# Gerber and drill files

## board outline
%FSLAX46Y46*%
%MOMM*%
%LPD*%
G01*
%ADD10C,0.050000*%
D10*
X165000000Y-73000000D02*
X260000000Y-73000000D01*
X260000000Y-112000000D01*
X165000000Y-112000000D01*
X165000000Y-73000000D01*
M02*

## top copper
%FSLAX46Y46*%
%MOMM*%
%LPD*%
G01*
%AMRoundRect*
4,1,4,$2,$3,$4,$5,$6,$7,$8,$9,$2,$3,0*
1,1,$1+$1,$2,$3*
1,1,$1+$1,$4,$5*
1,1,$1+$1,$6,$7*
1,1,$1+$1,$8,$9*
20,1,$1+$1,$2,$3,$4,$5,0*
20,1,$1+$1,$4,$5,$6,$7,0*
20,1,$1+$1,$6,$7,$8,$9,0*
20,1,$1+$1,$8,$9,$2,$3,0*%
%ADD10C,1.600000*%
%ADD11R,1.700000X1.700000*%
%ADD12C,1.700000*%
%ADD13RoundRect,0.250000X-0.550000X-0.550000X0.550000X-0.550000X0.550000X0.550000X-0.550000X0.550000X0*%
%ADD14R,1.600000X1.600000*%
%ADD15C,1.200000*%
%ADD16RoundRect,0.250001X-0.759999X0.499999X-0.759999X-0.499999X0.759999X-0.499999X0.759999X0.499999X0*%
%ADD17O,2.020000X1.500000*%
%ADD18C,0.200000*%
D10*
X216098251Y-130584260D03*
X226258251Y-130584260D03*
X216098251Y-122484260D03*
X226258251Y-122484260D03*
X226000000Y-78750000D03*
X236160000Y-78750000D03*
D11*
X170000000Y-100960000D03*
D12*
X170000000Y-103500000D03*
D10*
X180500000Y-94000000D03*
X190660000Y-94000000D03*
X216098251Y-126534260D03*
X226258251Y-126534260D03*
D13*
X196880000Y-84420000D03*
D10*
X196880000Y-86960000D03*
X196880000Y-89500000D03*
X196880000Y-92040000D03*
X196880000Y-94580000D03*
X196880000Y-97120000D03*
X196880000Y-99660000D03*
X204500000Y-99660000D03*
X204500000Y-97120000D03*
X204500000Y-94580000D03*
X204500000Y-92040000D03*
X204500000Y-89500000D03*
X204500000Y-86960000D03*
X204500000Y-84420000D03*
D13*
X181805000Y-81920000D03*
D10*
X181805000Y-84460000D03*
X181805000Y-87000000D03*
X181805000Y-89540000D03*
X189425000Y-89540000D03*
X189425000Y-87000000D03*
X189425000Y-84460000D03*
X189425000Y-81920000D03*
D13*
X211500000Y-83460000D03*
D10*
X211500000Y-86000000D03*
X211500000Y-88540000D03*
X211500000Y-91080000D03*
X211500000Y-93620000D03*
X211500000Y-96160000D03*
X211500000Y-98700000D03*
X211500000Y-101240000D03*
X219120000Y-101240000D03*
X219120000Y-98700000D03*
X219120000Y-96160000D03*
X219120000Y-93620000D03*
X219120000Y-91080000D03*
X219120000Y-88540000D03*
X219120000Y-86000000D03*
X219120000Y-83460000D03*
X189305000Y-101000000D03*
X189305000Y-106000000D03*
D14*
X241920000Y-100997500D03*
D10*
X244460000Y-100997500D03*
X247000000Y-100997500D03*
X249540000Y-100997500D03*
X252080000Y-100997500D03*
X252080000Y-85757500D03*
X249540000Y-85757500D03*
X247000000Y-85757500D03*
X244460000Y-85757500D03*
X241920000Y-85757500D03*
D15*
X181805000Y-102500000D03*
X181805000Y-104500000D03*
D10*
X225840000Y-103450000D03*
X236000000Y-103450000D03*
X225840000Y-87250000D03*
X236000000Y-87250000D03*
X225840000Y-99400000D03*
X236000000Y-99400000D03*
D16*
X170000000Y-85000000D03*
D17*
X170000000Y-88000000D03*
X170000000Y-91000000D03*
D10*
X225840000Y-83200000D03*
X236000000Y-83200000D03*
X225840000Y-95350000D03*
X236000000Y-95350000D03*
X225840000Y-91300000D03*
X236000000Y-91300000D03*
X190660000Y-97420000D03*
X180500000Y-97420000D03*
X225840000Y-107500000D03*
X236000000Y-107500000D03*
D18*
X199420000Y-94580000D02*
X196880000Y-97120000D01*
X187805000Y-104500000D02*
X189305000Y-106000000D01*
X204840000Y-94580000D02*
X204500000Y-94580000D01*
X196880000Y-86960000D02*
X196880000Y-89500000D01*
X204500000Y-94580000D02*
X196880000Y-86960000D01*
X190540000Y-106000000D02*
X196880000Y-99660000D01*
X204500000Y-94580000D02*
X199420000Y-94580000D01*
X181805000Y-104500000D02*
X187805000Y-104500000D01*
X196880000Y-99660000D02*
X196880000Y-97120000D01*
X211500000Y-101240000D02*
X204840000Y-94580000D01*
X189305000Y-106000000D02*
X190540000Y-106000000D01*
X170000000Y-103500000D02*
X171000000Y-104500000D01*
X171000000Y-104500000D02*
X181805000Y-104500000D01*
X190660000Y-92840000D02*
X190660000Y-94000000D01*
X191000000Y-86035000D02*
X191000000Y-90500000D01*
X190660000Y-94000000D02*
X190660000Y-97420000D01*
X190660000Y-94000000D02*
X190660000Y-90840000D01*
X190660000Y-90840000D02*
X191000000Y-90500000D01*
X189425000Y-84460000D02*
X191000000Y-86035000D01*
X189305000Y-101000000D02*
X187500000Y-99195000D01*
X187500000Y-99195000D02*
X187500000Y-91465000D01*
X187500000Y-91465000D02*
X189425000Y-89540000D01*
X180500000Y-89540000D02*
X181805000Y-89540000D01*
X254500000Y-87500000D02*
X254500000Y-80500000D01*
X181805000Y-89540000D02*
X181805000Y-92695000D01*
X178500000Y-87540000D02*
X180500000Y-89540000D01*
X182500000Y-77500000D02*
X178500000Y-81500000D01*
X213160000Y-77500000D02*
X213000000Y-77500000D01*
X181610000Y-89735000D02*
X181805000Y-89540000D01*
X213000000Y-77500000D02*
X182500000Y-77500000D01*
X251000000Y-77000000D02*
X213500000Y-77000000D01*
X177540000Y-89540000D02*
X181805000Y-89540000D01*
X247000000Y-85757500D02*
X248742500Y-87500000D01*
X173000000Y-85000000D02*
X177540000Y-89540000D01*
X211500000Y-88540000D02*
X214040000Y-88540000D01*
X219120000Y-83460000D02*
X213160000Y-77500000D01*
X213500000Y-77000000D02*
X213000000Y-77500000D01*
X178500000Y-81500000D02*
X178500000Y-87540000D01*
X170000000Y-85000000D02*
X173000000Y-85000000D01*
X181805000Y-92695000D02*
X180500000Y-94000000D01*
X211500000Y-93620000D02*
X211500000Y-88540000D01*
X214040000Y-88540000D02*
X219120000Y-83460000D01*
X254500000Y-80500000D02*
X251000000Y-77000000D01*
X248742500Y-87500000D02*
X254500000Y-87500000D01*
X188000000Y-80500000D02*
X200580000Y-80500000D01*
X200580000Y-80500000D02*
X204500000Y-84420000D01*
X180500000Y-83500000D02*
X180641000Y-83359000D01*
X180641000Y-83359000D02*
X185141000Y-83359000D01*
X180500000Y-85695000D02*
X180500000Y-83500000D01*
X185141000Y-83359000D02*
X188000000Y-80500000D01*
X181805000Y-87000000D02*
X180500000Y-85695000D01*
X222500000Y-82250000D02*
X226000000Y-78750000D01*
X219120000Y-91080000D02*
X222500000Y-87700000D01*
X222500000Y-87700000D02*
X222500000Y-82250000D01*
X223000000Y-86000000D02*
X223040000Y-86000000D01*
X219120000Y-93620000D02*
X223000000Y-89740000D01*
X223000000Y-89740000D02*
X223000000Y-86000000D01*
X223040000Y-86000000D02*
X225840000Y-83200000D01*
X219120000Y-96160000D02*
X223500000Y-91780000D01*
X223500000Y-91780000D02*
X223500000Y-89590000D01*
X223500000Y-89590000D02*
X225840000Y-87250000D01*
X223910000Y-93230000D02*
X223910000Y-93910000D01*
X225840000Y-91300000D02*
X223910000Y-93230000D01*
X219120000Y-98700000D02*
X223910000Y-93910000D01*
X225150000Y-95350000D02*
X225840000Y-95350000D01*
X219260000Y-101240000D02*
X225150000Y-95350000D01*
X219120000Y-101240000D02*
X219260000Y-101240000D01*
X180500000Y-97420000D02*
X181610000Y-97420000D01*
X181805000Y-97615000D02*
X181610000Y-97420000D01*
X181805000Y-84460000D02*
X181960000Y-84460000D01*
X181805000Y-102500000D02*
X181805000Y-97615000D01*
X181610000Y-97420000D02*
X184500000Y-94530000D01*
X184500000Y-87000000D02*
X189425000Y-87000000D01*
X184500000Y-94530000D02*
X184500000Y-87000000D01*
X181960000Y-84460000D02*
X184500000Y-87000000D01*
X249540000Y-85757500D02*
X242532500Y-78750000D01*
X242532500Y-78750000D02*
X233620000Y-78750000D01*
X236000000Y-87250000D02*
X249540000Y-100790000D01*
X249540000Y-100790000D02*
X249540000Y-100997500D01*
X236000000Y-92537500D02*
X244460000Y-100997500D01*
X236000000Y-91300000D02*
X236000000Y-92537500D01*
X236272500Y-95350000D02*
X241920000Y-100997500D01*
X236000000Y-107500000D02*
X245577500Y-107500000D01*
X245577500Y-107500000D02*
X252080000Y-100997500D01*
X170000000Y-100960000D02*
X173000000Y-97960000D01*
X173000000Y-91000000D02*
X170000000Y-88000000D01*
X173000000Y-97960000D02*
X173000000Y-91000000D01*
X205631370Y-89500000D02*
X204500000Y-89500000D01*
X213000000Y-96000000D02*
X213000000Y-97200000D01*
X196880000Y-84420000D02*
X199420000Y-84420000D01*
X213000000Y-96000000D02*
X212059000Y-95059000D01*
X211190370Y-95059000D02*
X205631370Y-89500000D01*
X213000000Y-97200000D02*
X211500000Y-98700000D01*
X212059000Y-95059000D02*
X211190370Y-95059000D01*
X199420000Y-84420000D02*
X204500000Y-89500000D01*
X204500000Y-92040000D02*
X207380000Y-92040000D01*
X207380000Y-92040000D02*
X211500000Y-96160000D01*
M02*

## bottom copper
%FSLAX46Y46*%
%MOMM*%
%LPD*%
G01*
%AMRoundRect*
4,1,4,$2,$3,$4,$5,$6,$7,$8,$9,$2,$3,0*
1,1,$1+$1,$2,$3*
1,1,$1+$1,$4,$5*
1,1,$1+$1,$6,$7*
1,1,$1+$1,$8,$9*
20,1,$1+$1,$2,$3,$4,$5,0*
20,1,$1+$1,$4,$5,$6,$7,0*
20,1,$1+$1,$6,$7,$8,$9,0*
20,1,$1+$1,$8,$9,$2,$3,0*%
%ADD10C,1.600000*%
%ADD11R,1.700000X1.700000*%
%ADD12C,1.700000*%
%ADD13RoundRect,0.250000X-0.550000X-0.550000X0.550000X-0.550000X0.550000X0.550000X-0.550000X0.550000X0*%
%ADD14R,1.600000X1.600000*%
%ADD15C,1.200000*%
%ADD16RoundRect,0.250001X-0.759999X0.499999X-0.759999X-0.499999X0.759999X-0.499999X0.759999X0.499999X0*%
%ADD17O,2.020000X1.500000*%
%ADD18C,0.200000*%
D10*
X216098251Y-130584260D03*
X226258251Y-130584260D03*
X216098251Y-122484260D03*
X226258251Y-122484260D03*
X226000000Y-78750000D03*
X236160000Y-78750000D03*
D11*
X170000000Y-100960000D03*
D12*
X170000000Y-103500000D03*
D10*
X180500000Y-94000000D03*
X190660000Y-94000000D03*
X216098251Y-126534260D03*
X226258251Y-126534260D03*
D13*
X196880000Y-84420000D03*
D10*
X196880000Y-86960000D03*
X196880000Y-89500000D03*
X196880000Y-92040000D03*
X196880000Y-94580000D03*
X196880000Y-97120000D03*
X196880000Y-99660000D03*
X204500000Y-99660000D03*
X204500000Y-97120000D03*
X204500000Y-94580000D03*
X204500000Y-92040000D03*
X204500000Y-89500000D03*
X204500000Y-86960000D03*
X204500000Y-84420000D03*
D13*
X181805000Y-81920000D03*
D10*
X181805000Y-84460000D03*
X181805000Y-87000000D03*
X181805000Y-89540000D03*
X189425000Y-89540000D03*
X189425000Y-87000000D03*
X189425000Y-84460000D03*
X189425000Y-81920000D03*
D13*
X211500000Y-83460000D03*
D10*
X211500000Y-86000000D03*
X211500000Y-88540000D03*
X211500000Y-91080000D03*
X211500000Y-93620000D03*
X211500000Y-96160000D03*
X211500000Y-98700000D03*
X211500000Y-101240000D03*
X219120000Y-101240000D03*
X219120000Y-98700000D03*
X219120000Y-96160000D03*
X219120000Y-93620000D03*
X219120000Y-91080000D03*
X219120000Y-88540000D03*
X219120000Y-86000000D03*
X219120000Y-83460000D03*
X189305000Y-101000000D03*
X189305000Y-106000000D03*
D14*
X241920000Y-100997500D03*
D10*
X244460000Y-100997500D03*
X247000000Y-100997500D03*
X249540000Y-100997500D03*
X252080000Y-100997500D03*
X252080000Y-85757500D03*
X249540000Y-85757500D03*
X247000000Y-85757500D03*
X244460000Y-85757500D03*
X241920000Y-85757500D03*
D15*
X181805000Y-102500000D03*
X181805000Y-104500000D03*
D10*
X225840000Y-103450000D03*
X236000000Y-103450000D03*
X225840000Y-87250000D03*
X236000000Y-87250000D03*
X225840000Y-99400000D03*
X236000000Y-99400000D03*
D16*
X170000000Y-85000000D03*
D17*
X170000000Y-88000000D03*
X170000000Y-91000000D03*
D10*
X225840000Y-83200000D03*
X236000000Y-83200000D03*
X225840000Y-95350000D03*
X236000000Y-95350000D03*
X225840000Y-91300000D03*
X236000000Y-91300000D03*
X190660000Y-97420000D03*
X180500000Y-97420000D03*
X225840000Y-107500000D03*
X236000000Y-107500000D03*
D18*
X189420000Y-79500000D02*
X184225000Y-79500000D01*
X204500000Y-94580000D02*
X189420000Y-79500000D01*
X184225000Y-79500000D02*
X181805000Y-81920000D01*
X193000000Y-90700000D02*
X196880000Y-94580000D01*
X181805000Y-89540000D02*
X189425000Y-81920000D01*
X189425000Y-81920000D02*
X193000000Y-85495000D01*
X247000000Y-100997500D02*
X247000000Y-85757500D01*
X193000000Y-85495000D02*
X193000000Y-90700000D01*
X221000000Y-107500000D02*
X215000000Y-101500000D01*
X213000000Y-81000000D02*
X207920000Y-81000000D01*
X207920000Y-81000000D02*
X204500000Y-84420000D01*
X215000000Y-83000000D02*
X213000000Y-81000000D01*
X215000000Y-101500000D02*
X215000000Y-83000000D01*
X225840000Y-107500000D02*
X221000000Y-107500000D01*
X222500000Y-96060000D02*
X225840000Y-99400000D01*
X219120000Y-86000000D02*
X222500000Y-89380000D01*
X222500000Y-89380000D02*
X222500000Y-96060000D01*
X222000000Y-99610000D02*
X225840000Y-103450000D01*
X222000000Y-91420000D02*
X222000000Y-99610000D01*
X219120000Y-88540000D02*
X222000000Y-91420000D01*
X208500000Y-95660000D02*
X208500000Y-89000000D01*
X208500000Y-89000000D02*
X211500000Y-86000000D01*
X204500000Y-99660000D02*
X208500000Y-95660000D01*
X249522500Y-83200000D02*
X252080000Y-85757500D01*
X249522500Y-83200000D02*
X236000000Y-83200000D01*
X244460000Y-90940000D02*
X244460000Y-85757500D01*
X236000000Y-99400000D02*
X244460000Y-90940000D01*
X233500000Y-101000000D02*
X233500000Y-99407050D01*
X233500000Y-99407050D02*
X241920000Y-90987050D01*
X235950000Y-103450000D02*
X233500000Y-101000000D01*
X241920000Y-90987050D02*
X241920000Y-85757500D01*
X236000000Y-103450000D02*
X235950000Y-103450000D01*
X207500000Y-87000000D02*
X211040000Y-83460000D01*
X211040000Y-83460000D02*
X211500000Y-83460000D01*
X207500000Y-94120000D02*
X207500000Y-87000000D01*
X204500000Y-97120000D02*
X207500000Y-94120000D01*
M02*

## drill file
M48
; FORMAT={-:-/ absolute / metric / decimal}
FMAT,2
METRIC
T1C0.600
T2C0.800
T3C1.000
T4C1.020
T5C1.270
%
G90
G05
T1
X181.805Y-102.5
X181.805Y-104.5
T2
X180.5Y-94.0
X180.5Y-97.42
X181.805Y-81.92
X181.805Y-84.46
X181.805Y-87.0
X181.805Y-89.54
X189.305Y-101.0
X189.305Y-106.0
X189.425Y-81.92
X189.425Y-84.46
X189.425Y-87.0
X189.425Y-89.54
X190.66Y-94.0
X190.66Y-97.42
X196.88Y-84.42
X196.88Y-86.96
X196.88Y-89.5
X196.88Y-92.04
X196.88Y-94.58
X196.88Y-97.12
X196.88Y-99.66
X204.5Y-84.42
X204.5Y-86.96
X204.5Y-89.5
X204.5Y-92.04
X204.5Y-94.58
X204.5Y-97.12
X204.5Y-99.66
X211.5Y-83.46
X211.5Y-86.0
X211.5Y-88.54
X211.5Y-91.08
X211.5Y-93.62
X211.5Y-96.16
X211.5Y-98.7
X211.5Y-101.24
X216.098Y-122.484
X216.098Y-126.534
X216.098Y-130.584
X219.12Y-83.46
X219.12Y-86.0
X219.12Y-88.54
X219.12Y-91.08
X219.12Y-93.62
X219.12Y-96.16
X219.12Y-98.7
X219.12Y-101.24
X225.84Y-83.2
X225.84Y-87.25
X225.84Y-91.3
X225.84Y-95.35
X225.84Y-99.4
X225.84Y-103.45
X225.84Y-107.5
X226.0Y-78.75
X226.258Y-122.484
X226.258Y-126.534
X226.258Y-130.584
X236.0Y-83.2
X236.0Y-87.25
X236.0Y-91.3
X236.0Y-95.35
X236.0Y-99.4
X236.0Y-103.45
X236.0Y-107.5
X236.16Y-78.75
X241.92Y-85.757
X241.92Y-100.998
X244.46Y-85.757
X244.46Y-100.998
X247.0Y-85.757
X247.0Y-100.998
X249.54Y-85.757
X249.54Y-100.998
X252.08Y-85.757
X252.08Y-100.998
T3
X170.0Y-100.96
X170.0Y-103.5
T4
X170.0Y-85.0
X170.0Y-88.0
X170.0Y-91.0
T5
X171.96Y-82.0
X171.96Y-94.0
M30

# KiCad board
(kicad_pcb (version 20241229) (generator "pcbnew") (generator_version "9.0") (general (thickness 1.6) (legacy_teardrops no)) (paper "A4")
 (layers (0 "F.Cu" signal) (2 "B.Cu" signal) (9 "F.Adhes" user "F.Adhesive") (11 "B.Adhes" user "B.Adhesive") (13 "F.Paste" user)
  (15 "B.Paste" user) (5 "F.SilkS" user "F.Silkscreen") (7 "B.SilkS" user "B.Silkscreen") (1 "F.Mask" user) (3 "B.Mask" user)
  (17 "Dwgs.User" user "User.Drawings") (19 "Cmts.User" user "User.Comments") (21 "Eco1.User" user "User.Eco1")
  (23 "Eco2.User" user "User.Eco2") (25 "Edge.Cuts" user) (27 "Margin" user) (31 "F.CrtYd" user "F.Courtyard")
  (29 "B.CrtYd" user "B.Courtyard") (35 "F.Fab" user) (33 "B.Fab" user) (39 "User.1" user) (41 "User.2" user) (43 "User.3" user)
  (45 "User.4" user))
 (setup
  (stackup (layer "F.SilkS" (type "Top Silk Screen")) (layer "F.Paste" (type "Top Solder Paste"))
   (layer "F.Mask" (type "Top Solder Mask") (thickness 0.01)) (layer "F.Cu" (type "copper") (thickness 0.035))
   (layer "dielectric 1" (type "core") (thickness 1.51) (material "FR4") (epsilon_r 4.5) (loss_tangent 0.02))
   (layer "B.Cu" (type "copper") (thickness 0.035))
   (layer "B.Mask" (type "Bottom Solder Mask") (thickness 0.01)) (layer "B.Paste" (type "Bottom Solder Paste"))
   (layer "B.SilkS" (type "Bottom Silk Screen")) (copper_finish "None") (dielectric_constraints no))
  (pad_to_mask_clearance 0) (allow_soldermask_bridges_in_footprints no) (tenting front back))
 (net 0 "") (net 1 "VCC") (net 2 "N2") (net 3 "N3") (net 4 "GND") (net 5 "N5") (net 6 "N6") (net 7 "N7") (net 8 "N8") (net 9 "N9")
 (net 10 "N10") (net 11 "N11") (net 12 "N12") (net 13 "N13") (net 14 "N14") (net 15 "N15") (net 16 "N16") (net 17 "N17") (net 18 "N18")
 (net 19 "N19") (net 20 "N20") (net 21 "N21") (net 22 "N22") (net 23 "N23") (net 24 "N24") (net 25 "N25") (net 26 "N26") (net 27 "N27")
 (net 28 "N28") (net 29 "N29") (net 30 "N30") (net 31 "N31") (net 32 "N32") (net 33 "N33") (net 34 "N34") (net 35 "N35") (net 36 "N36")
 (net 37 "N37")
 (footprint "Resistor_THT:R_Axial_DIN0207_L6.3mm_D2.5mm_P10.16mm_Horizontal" (layer "F.Cu") (at 216.098251 130.58426)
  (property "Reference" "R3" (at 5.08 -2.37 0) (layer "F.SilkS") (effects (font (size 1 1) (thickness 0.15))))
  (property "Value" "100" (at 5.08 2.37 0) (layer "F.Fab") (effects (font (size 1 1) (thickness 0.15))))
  (pad "1" thru_hole circle (at 0 0) (size 1.6 1.6) (drill 0.8) (layers "*.Cu" "*.Mask") (remove_unused_layers no) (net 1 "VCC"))
  (pad "2" thru_hole circle (at 10.16 0) (size 1.6 1.6) (drill 0.8) (layers "*.Cu" "*.Mask") (remove_unused_layers no) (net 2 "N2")))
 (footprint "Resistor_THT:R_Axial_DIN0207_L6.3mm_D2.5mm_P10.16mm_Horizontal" (layer "F.Cu") (at 216.098251 122.48426)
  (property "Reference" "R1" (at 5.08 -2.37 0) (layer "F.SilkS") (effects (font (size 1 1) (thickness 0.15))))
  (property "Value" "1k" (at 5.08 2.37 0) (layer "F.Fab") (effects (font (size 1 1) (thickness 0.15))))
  (pad "1" thru_hole circle (at 0 0) (size 1.6 1.6) (drill 0.8) (layers "*.Cu" "*.Mask") (remove_unused_layers no) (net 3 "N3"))
  (pad "2" thru_hole circle (at 10.16 0) (size 1.6 1.6) (drill 0.8) (layers "*.Cu" "*.Mask") (remove_unused_layers no) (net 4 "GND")))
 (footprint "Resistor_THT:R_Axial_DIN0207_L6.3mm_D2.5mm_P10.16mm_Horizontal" (layer "F.Cu") (at 226 78.75)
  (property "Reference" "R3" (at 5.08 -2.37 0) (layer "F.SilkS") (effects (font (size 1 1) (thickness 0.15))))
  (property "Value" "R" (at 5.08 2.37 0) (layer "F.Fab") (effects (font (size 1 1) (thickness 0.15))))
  (pad "1" thru_hole circle (at 0 0) (size 1.6 1.6) (drill 0.8) (layers "*.Cu" "*.Mask") (remove_unused_layers no) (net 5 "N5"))
  (pad "2" thru_hole circle (at 10.16 0) (size 1.6 1.6) (drill 0.8) (layers "*.Cu" "*.Mask") (remove_unused_layers no) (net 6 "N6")))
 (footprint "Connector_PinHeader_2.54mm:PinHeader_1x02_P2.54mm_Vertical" (layer "F.Cu") (at 170 100.96)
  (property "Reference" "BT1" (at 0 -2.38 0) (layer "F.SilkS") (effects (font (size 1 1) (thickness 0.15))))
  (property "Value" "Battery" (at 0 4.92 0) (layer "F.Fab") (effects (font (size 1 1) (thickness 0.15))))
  (pad "1" thru_hole rect (at 0 0) (size 1.7 1.7) (drill 1) (layers "*.Cu" "*.Mask") (remove_unused_layers no) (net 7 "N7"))
  (pad "2" thru_hole circle (at 0 2.54) (size 1.7 1.7) (drill 1) (layers "*.Cu" "*.Mask") (remove_unused_layers no) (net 4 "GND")))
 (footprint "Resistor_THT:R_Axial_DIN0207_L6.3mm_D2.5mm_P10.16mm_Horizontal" (layer "F.Cu") (at 180.5 94)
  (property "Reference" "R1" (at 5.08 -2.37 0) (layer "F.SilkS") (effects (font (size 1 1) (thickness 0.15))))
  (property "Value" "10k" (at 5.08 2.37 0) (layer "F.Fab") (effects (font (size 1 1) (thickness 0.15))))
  (pad "1" thru_hole circle (at 0 0) (size 1.6 1.6) (drill 0.8) (layers "*.Cu" "*.Mask") (remove_unused_layers no) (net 1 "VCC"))
  (pad "2" thru_hole circle (at 10.16 0) (size 1.6 1.6) (drill 0.8) (layers "*.Cu" "*.Mask") (remove_unused_layers no) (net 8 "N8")))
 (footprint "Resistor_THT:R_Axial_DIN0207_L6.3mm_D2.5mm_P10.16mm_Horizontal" (layer "F.Cu") (at 216.098251 126.53426)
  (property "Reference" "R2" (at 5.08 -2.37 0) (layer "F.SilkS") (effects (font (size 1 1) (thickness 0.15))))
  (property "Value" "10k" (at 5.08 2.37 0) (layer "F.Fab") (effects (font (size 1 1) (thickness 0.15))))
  (pad "1" thru_hole circle (at 0 0) (size 1.6 1.6) (drill 0.8) (layers "*.Cu" "*.Mask") (remove_unused_layers no) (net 1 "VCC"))
  (pad "2" thru_hole circle (at 10.16 0) (size 1.6 1.6) (drill 0.8) (layers "*.Cu" "*.Mask") (remove_unused_layers no) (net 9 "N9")))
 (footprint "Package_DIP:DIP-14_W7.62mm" (layer "F.Cu") (at 196.88 84.42)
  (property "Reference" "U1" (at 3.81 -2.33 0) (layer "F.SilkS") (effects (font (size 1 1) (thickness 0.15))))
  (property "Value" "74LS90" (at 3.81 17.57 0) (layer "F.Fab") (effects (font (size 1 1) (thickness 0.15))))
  (pad "1" thru_hole roundrect (at 0 0) (size 1.6 1.6) (drill 0.8) (layers "*.Cu" "*.Mask") (remove_unused_layers no)
   (roundrect_rratio 0.15625) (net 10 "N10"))
  (pad "2" thru_hole circle (at 0 2.54) (size 1.6 1.6) (drill 0.8) (layers "*.Cu" "*.Mask") (remove_unused_layers no) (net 4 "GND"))
  (pad "3" thru_hole circle (at 0 5.08) (size 1.6 1.6) (drill 0.8) (layers "*.Cu" "*.Mask") (remove_unused_layers no) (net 4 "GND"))
  (pad "4" thru_hole circle (at 0 7.62) (size 1.6 1.6) (drill 0.8) (layers "*.Cu" "*.Mask") (remove_unused_layers no))
  (pad "5" thru_hole circle (at 0 10.16) (size 1.6 1.6) (drill 0.8) (layers "*.Cu" "*.Mask") (remove_unused_layers no) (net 1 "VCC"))
  (pad "6" thru_hole circle (at 0 12.7) (size 1.6 1.6) (drill 0.8) (layers "*.Cu" "*.Mask") (remove_unused_layers no) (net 4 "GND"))
  (pad "7" thru_hole circle (at 0 15.24) (size 1.6 1.6) (drill 0.8) (layers "*.Cu" "*.Mask") (remove_unused_layers no) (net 4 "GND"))
  (pad "8" thru_hole circle (at 7.62 15.24) (size 1.6 1.6) (drill 0.8) (layers "*.Cu" "*.Mask") (remove_unused_layers no) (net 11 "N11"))
  (pad "9" thru_hole circle (at 7.62 12.7) (size 1.6 1.6) (drill 0.8) (layers "*.Cu" "*.Mask") (remove_unused_layers no) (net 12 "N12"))
  (pad "10" thru_hole circle (at 7.62 10.16) (size 1.6 1.6) (drill 0.8) (layers "*.Cu" "*.Mask") (remove_unused_layers no) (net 4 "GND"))
  (pad "11" thru_hole circle (at 7.62 7.62) (size 1.6 1.6) (drill 0.8) (layers "*.Cu" "*.Mask") (remove_unused_layers no) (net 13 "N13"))
  (pad "12" thru_hole circle (at 7.62 5.08) (size 1.6 1.6) (drill 0.8) (layers "*.Cu" "*.Mask") (remove_unused_layers no) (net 10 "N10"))
  (pad "13" thru_hole circle (at 7.62 2.54) (size 1.6 1.6) (drill 0.8) (layers "*.Cu" "*.Mask") (remove_unused_layers no))
  (pad "14" thru_hole circle (at 7.62 0) (size 1.6 1.6) (drill 0.8) (layers "*.Cu" "*.Mask") (remove_unused_layers no) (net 9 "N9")))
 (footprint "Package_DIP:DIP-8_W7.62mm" (layer "F.Cu") (at 181.805 81.92)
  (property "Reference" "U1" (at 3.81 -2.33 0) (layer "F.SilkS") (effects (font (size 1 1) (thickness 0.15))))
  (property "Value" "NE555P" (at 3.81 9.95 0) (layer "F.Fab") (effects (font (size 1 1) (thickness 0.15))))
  (pad "1" thru_hole roundrect (at 0 0) (size 1.6 1.6) (drill 0.8) (layers "*.Cu" "*.Mask") (remove_unused_layers no)
   (roundrect_rratio 0.15625) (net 4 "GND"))
  (pad "2" thru_hole circle (at 0 2.54) (size 1.6 1.6) (drill 0.8) (layers "*.Cu" "*.Mask") (remove_unused_layers no) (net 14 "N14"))
  (pad "3" thru_hole circle (at 0 5.08) (size 1.6 1.6) (drill 0.8) (layers "*.Cu" "*.Mask") (remove_unused_layers no) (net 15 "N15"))
  (pad "4" thru_hole circle (at 0 7.62) (size 1.6 1.6) (drill 0.8) (layers "*.Cu" "*.Mask") (remove_unused_layers no) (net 1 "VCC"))
  (pad "5" thru_hole circle (at 7.62 7.62) (size 1.6 1.6) (drill 0.8) (layers "*.Cu" "*.Mask") (remove_unused_layers no) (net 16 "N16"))
  (pad "6" thru_hole circle (at 7.62 5.08) (size 1.6 1.6) (drill 0.8) (layers "*.Cu" "*.Mask") (remove_unused_layers no) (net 14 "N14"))
  (pad "7" thru_hole circle (at 7.62 2.54) (size 1.6 1.6) (drill 0.8) (layers "*.Cu" "*.Mask") (remove_unused_layers no) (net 8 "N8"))
  (pad "8" thru_hole circle (at 7.62 0) (size 1.6 1.6) (drill 0.8) (layers "*.Cu" "*.Mask") (remove_unused_layers no) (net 1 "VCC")))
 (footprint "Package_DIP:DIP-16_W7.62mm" (layer "F.Cu") (at 211.5 83.46)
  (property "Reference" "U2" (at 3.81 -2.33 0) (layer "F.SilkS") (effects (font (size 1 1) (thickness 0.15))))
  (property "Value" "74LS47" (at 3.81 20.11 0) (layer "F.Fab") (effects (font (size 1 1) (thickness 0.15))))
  (pad "1" thru_hole roundrect (at 0 0) (size 1.6 1.6) (drill 0.8) (layers "*.Cu" "*.Mask") (remove_unused_layers no)
   (roundrect_rratio 0.15625) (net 12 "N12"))
  (pad "2" thru_hole circle (at 0 2.54) (size 1.6 1.6) (drill 0.8) (layers "*.Cu" "*.Mask") (remove_unused_layers no) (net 11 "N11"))
  (pad "3" thru_hole circle (at 0 5.08) (size 1.6 1.6) (drill 0.8) (layers "*.Cu" "*.Mask") (remove_unused_layers no) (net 1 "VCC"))
  (pad "4" thru_hole circle (at 0 7.62) (size 1.6 1.6) (drill 0.8) (layers "*.Cu" "*.Mask") (remove_unused_layers no) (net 1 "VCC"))
  (pad "5" thru_hole circle (at 0 10.16) (size 1.6 1.6) (drill 0.8) (layers "*.Cu" "*.Mask") (remove_unused_layers no) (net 1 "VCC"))
  (pad "6" thru_hole circle (at 0 12.7) (size 1.6 1.6) (drill 0.8) (layers "*.Cu" "*.Mask") (remove_unused_layers no) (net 13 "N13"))
  (pad "7" thru_hole circle (at 0 15.24) (size 1.6 1.6) (drill 0.8) (layers "*.Cu" "*.Mask") (remove_unused_layers no) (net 10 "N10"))
  (pad "8" thru_hole circle (at 0 17.78) (size 1.6 1.6) (drill 0.8) (layers "*.Cu" "*.Mask") (remove_unused_layers no) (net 4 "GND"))
  (pad "9" thru_hole circle (at 7.62 17.78) (size 1.6 1.6) (drill 0.8) (layers "*.Cu" "*.Mask") (remove_unused_layers no) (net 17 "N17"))
  (pad "10" thru_hole circle (at 7.62 15.24) (size 1.6 1.6) (drill 0.8) (layers "*.Cu" "*.Mask") (remove_unused_layers no) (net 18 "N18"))
  (pad "11" thru_hole circle (at 7.62 12.7) (size 1.6 1.6) (drill 0.8) (layers "*.Cu" "*.Mask") (remove_unused_layers no) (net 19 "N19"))
  (pad "12" thru_hole circle (at 7.62 10.16) (size 1.6 1.6) (drill 0.8) (layers "*.Cu" "*.Mask") (remove_unused_layers no) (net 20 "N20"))
  (pad "13" thru_hole circle (at 7.62 7.62) (size 1.6 1.6) (drill 0.8) (layers "*.Cu" "*.Mask") (remove_unused_layers no) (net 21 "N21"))
  (pad "14" thru_hole circle (at 7.62 5.08) (size 1.6 1.6) (drill 0.8) (layers "*.Cu" "*.Mask") (remove_unused_layers no) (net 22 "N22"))
  (pad "15" thru_hole circle (at 7.62 2.54) (size 1.6 1.6) (drill 0.8) (layers "*.Cu" "*.Mask") (remove_unused_layers no) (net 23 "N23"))
  (pad "16" thru_hole circle (at 7.62 0) (size 1.6 1.6) (drill 0.8) (layers "*.Cu" "*.Mask") (remove_unused_layers no) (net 1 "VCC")))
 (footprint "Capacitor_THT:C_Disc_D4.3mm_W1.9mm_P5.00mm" (layer "F.Cu") (at 189.305 101 -90)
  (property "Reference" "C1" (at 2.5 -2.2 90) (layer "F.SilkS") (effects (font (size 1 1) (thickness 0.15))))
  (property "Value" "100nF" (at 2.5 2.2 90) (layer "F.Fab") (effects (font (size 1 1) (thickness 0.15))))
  (pad "1" thru_hole circle (at 0 0 270) (size 1.6 1.6) (drill 0.8) (layers "*.Cu" "*.Mask") (remove_unused_layers no) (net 9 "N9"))
  (pad "2" thru_hole circle (at 5 0 270) (size 1.6 1.6) (drill 0.8) (layers "*.Cu" "*.Mask") (remove_unused_layers no) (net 3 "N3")))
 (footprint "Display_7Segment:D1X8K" (layer "F.Cu") (at 241.92 100.9975 90)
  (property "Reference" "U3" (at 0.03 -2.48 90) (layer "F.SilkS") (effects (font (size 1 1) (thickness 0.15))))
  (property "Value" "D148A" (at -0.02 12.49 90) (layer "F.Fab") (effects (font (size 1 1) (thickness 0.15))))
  (pad "1" thru_hole rect (at 0 0) (size 1.6 1.6) (drill 0.8) (layers "*.Cu" "*.Mask") (remove_unused_layers no) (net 17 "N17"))
  (pad "2" thru_hole circle (at 0 2.54) (size 1.6 1.6) (drill 0.8) (layers "*.Cu" "*.Mask") (remove_unused_layers no) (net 18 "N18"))
  (pad "3" thru_hole circle (at 0 5.08) (size 1.6 1.6) (drill 0.8) (layers "*.Cu" "*.Mask") (remove_unused_layers no) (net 2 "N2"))
  (pad "4" thru_hole circle (at 0 7.62) (size 1.6 1.6) (drill 0.8) (layers "*.Cu" "*.Mask") (remove_unused_layers no) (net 19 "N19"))
  (pad "5" thru_hole circle (at 0 10.16) (size 1.6 1.6) (drill 0.8) (layers "*.Cu" "*.Mask") (remove_unused_layers no) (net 9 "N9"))
  (pad "6" thru_hole circle (at 15.24 10.16) (size 1.6 1.6) (drill 0.8) (layers "*.Cu" "*.Mask") (remove_unused_layers no) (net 20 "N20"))
  (pad "7" thru_hole circle (at 15.24 7.62) (size 1.6 1.6) (drill 0.8) (layers "*.Cu" "*.Mask") (remove_unused_layers no) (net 21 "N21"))
  (pad "8" thru_hole circle (at 15.24 5.08) (size 1.6 1.6) (drill 0.8) (layers "*.Cu" "*.Mask") (remove_unused_layers no) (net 2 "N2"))
  (pad "9" thru_hole circle (at 15.24 2.54) (size 1.6 1.6) (drill 0.8) (layers "*.Cu" "*.Mask") (remove_unused_layers no) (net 23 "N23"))
  (pad "10" thru_hole circle (at 15.24 0) (size 1.6 1.6) (drill 0.8) (layers "*.Cu" "*.Mask") (remove_unused_layers no) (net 22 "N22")))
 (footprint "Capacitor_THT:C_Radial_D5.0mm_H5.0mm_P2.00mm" (layer "F.Cu") (at 181.805 102.5 -90)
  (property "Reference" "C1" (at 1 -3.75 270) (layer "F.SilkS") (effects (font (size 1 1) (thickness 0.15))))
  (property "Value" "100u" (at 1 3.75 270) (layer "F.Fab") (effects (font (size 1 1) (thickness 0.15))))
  (pad "1" thru_hole circle (at 0 0 270) (size 1.2 1.2) (drill 0.6) (layers "*.Cu" "*.Mask") (remove_unused_layers no) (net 14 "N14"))
  (pad "2" thru_hole circle (at 2 0 270) (size 1.2 1.2) (drill 0.6) (layers "*.Cu" "*.Mask") (remove_unused_layers no) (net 4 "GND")))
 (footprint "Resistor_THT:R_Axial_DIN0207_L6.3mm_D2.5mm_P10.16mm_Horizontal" (layer "F.Cu") (at 225.84 103.45)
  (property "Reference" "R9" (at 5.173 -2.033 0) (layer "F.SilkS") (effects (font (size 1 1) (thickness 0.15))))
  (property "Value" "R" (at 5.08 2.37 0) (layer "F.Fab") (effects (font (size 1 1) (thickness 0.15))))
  (pad "1" thru_hole circle (at 0 0) (size 1.6 1.6) (drill 0.8) (layers "*.Cu" "*.Mask") (remove_unused_layers no) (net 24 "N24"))
  (pad "2" thru_hole circle (at 10.16 0) (size 1.6 1.6) (drill 0.8) (layers "*.Cu" "*.Mask") (remove_unused_layers no) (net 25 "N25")))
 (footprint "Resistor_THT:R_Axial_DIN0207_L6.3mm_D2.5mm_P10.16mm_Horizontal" (layer "F.Cu") (at 225.84 87.25)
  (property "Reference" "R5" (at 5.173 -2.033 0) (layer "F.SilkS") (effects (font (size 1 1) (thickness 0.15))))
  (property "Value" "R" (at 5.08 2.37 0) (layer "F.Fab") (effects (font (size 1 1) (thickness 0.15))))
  (pad "1" thru_hole circle (at 0 0) (size 1.6 1.6) (drill 0.8) (layers "*.Cu" "*.Mask") (remove_unused_layers no) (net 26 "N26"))
  (pad "2" thru_hole circle (at 10.16 0) (size 1.6 1.6) (drill 0.8) (layers "*.Cu" "*.Mask") (remove_unused_layers no) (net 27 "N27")))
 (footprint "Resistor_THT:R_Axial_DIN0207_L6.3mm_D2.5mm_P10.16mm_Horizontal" (layer "F.Cu") (at 225.84 99.4)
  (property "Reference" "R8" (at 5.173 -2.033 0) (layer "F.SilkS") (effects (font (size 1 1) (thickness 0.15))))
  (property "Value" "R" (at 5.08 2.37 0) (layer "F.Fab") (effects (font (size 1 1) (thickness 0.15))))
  (pad "1" thru_hole circle (at 0 0) (size 1.6 1.6) (drill 0.8) (layers "*.Cu" "*.Mask") (remove_unused_layers no) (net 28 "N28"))
  (pad "2" thru_hole circle (at 10.16 0) (size 1.6 1.6) (drill 0.8) (layers "*.Cu" "*.Mask") (remove_unused_layers no) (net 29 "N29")))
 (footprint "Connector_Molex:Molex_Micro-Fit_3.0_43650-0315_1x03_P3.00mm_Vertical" (layer "F.Cu") (at 170 85 -90)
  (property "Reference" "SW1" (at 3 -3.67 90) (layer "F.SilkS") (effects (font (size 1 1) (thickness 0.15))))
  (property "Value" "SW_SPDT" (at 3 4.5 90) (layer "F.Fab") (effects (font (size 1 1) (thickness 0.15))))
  (pad "" np_thru_hole circle (at -3 -1.96 270) (size 1.27 1.27) (drill 1.27) (layers "*.Cu" "*.Mask"))
  (pad "" np_thru_hole circle (at 9 -1.96 270) (size 1.27 1.27) (drill 1.27) (layers "*.Cu" "*.Mask"))
  (pad "1" thru_hole roundrect (at 0 0 270) (size 1.5 2.02) (drill 1.02) (layers "*.Cu" "*.Mask") (remove_unused_layers no)
   (roundrect_rratio 0.166667) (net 1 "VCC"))
  (pad "2" thru_hole oval (at 3 0 270) (size 1.5 2.02) (drill 1.02) (layers "*.Cu" "*.Mask") (remove_unused_layers no) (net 7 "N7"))
  (pad "3" thru_hole oval (at 6 0 270) (size 1.5 2.02) (drill 1.02) (layers "*.Cu" "*.Mask") (remove_unused_layers no) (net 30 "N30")))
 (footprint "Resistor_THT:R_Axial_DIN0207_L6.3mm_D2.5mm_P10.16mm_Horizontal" (layer "F.Cu") (at 225.84 83.2)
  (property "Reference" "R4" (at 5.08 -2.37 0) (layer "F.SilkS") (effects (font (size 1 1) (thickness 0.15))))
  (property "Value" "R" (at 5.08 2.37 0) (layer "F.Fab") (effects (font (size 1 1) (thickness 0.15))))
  (pad "1" thru_hole circle (at 0 0) (size 1.6 1.6) (drill 0.8) (layers "*.Cu" "*.Mask") (remove_unused_layers no) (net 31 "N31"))
  (pad "2" thru_hole circle (at 10.16 0) (size 1.6 1.6) (drill 0.8) (layers "*.Cu" "*.Mask") (remove_unused_layers no) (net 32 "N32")))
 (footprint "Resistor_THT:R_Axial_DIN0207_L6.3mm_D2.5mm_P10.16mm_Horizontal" (layer "F.Cu") (at 225.84 95.35)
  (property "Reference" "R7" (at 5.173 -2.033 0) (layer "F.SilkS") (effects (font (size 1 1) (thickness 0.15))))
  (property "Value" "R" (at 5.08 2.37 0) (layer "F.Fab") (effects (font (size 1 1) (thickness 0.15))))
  (pad "1" thru_hole circle (at 0 0) (size 1.6 1.6) (drill 0.8) (layers "*.Cu" "*.Mask") (remove_unused_layers no) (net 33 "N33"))
  (pad "2" thru_hole circle (at 10.16 0) (size 1.6 1.6) (drill 0.8) (layers "*.Cu" "*.Mask") (remove_unused_layers no) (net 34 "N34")))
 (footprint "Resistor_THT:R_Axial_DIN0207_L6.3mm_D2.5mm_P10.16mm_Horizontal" (layer "F.Cu") (at 225.84 91.3)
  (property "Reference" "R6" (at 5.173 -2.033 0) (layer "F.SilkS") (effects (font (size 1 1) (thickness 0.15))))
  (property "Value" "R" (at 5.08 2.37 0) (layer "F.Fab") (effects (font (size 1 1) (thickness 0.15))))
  (pad "1" thru_hole circle (at 0 0) (size 1.6 1.6) (drill 0.8) (layers "*.Cu" "*.Mask") (remove_unused_layers no) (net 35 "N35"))
  (pad "2" thru_hole circle (at 10.16 0) (size 1.6 1.6) (drill 0.8) (layers "*.Cu" "*.Mask") (remove_unused_layers no) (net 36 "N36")))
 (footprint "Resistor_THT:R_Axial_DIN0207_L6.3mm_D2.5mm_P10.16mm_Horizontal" (layer "F.Cu") (at 190.66 97.42 180)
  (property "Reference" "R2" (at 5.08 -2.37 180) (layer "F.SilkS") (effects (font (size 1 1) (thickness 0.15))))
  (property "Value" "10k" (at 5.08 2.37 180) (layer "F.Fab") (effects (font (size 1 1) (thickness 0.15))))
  (pad "1" thru_hole circle (at 0 0 180) (size 1.6 1.6) (drill 0.8) (layers "*.Cu" "*.Mask") (remove_unused_layers no) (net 8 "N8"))
  (pad "2" thru_hole circle (at 10.16 0 180) (size 1.6 1.6) (drill 0.8) (layers "*.Cu" "*.Mask") (remove_unused_layers no) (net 14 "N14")))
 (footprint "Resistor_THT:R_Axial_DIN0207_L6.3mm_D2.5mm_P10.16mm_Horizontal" (layer "F.Cu") (at 225.84 107.5)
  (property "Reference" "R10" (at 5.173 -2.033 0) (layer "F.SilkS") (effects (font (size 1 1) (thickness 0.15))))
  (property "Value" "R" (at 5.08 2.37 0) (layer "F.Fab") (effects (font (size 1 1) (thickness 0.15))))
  (pad "1" thru_hole circle (at 0 0) (size 1.6 1.6) (drill 0.8) (layers "*.Cu" "*.Mask") (remove_unused_layers no) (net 15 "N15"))
  (pad "2" thru_hole circle (at 10.16 0) (size 1.6 1.6) (drill 0.8) (layers "*.Cu" "*.Mask") (remove_unused_layers no) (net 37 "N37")))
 (gr_rect (start 165 73) (end 260 112) (stroke (width 0.05) (type default)) (fill no) (layer "Edge.Cuts"))
 (segment (start 199.42 94.58) (end 196.88 97.12) (width 0.2) (layer "F.Cu") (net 4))
 (segment (start 187.805 104.5) (end 189.305 106) (width 0.2) (layer "F.Cu") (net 4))
 (segment (start 204.84 94.58) (end 204.5 94.58) (width 0.2) (layer "F.Cu") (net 4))
 (segment (start 196.88 86.96) (end 196.88 89.5) (width 0.2) (layer "F.Cu") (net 4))
 (segment (start 204.5 94.58) (end 196.88 86.96) (width 0.2) (layer "F.Cu") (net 4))
 (segment (start 190.54 106) (end 196.88 99.66) (width 0.2) (layer "F.Cu") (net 4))
 (segment (start 204.5 94.58) (end 199.42 94.58) (width 0.2) (layer "F.Cu") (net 4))
 (segment (start 181.805 104.5) (end 187.805 104.5) (width 0.2) (layer "F.Cu") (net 4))
 (segment (start 196.88 99.66) (end 196.88 97.12) (width 0.2) (layer "F.Cu") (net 4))
 (segment (start 211.5 101.24) (end 204.84 94.58) (width 0.2) (layer "F.Cu") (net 4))
 (segment (start 189.305 106) (end 190.54 106) (width 0.2) (layer "F.Cu") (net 4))
 (segment (start 170 103.5) (end 171 104.5) (width 0.2) (layer "F.Cu") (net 4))
 (segment (start 171 104.5) (end 181.805 104.5) (width 0.2) (layer "F.Cu") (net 4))
 (segment (start 189.42 79.5) (end 184.225 79.5) (width 0.2) (layer "B.Cu") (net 4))
 (segment (start 204.5 94.58) (end 189.42 79.5) (width 0.2) (layer "B.Cu") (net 4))
 (segment (start 184.225 79.5) (end 181.805 81.92) (width 0.2) (layer "B.Cu") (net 4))
 (segment (start 190.66 92.84) (end 190.66 94) (width 0.2) (layer "F.Cu") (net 8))
 (segment (start 191 86.035) (end 191 90.5) (width 0.2) (layer "F.Cu") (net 8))
 (segment (start 190.66 94) (end 190.66 97.42) (width 0.2) (layer "F.Cu") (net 8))
 (segment (start 190.66 94) (end 190.66 90.84) (width 0.2) (layer "F.Cu") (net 8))
 (segment (start 190.66 90.84) (end 191 90.5) (width 0.2) (layer "F.Cu") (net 8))
 (segment (start 189.425 84.46) (end 191 86.035) (width 0.2) (layer "F.Cu") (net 8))
 (segment (start 189.305 101) (end 187.5 99.195) (width 0.2) (layer "F.Cu") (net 16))
 (segment (start 187.5 99.195) (end 187.5 91.465) (width 0.2) (layer "F.Cu") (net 16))
 (segment (start 187.5 91.465) (end 189.425 89.54) (width 0.2) (layer "F.Cu") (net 16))
 (segment (start 180.5 89.54) (end 181.805 89.54) (width 0.2) (layer "F.Cu") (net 1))
 (segment (start 254.5 87.5) (end 254.5 80.5) (width 0.2) (layer "F.Cu") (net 1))
 (segment (start 181.805 89.54) (end 181.805 92.695) (width 0.2) (layer "F.Cu") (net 1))
 (segment (start 178.5 87.54) (end 180.5 89.54) (width 0.2) (layer "F.Cu") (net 1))
 (segment (start 182.5 77.5) (end 178.5 81.5) (width 0.2) (layer "F.Cu") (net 1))
 (segment (start 213.16 77.5) (end 213 77.5) (width 0.2) (layer "F.Cu") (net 1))
 (segment (start 181.61 89.735) (end 181.805 89.54) (width 0.2) (layer "F.Cu") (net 1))
 (segment (start 213 77.5) (end 182.5 77.5) (width 0.2) (layer "F.Cu") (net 1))
 (segment (start 251 77) (end 213.5 77) (width 0.2) (layer "F.Cu") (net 1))
 (segment (start 177.54 89.54) (end 181.805 89.54) (width 0.2) (layer "F.Cu") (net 1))
 (segment (start 247 85.7575) (end 248.7425 87.5) (width 0.2) (layer "F.Cu") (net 1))
 (segment (start 173 85) (end 177.54 89.54) (width 0.2) (layer "F.Cu") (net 1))
 (segment (start 211.5 88.54) (end 214.04 88.54) (width 0.2) (layer "F.Cu") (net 1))
 (segment (start 219.12 83.46) (end 213.16 77.5) (width 0.2) (layer "F.Cu") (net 1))
 (segment (start 213.5 77) (end 213 77.5) (width 0.2) (layer "F.Cu") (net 1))
 (segment (start 178.5 81.5) (end 178.5 87.54) (width 0.2) (layer "F.Cu") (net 1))
 (segment (start 170 85) (end 173 85) (width 0.2) (layer "F.Cu") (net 1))
 (segment (start 181.805 92.695) (end 180.5 94) (width 0.2) (layer "F.Cu") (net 1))
 (segment (start 211.5 93.62) (end 211.5 88.54) (width 0.2) (layer "F.Cu") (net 1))
 (segment (start 214.04 88.54) (end 219.12 83.46) (width 0.2) (layer "F.Cu") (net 1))
 (segment (start 254.5 80.5) (end 251 77) (width 0.2) (layer "F.Cu") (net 1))
 (segment (start 248.7425 87.5) (end 254.5 87.5) (width 0.2) (layer "F.Cu") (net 1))
 (segment (start 193 90.7) (end 196.88 94.58) (width 0.2) (layer "B.Cu") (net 1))
 (segment (start 181.805 89.54) (end 189.425 81.92) (width 0.2) (layer "B.Cu") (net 1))
 (segment (start 189.425 81.92) (end 193 85.495) (width 0.2) (layer "B.Cu") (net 1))
 (segment (start 247 100.9975) (end 247 85.7575) (width 0.2) (layer "B.Cu") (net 1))
 (segment (start 193 85.495) (end 193 90.7) (width 0.2) (layer "B.Cu") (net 1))
 (segment (start 188 80.5) (end 200.58 80.5) (width 0.2) (layer "F.Cu") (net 15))
 (segment (start 200.58 80.5) (end 204.5 84.42) (width 0.2) (layer "F.Cu") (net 15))
 (segment (start 180.5 83.5) (end 180.641 83.359) (width 0.2) (layer "F.Cu") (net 15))
 (segment (start 180.641 83.359) (end 185.141 83.359) (width 0.2) (layer "F.Cu") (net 15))
 (segment (start 180.5 85.695) (end 180.5 83.5) (width 0.2) (layer "F.Cu") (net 15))
 (segment (start 185.141 83.359) (end 188 80.5) (width 0.2) (layer "F.Cu") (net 15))
 (segment (start 181.805 87) (end 180.5 85.695) (width 0.2) (layer "F.Cu") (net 15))
 (segment (start 221 107.5) (end 215 101.5) (width 0.2) (layer "B.Cu") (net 15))
 (segment (start 213 81) (end 207.92 81) (width 0.2) (layer "B.Cu") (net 15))
 (segment (start 207.92 81) (end 204.5 84.42) (width 0.2) (layer "B.Cu") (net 15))
 (segment (start 215 83) (end 213 81) (width 0.2) (layer "B.Cu") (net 15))
 (segment (start 215 101.5) (end 215 83) (width 0.2) (layer "B.Cu") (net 15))
 (segment (start 225.84 107.5) (end 221 107.5) (width 0.2) (layer "B.Cu") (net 15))
 (segment (start 222.5 82.25) (end 226 78.75) (width 0.2) (layer "F.Cu") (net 5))
 (segment (start 219.12 91.08) (end 222.5 87.7) (width 0.2) (layer "F.Cu") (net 5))
 (segment (start 222.5 87.7) (end 222.5 82.25) (width 0.2) (layer "F.Cu") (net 5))
 (segment (start 223 86) (end 223.04 86) (width 0.2) (layer "F.Cu") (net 31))
 (segment (start 219.12 93.62) (end 223 89.74) (width 0.2) (layer "F.Cu") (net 31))
 (segment (start 223 89.74) (end 223 86) (width 0.2) (layer "F.Cu") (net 31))
 (segment (start 223.04 86) (end 225.84 83.2) (width 0.2) (layer "F.Cu") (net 31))
 (segment (start 219.12 96.16) (end 223.5 91.78) (width 0.2) (layer "F.Cu") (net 26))
 (segment (start 223.5 91.78) (end 223.5 89.59) (width 0.2) (layer "F.Cu") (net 26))
 (segment (start 223.5 89.59) (end 225.84 87.25) (width 0.2) (layer "F.Cu") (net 26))
 (segment (start 223.91 93.23) (end 223.91 93.91) (width 0.2) (layer "F.Cu") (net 35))
 (segment (start 225.84 91.3) (end 223.91 93.23) (width 0.2) (layer "F.Cu") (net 35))
 (segment (start 219.12 98.7) (end 223.91 93.91) (width 0.2) (layer "F.Cu") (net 35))
 (segment (start 225.15 95.35) (end 225.84 95.35) (width 0.2) (layer "F.Cu") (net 33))
 (segment (start 219.26 101.24) (end 225.15 95.35) (width 0.2) (layer "F.Cu") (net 33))
 (segment (start 219.12 101.24) (end 219.26 101.24) (width 0.2) (layer "F.Cu") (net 33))
 (segment (start 222.5 96.06) (end 225.84 99.4) (width 0.2) (layer "B.Cu") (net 28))
 (segment (start 219.12 86) (end 222.5 89.38) (width 0.2) (layer "B.Cu") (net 28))
 (segment (start 222.5 89.38) (end 222.5 96.06) (width 0.2) (layer "B.Cu") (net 28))
 (segment (start 222 99.61) (end 225.84 103.45) (width 0.2) (layer "B.Cu") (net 24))
 (segment (start 222 91.42) (end 222 99.61) (width 0.2) (layer "B.Cu") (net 24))
 (segment (start 219.12 88.54) (end 222 91.42) (width 0.2) (layer "B.Cu") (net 24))
 (segment (start 208.5 95.66) (end 208.5 89) (width 0.2) (layer "B.Cu") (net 11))
 (segment (start 208.5 89) (end 211.5 86) (width 0.2) (layer "B.Cu") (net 11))
 (segment (start 204.5 99.66) (end 208.5 95.66) (width 0.2) (layer "B.Cu") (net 11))
 (segment (start 180.5 97.42) (end 181.61 97.42) (width 0.2) (layer "F.Cu") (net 14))
 (segment (start 181.805 97.615) (end 181.61 97.42) (width 0.2) (layer "F.Cu") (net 14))
 (segment (start 181.805 84.46) (end 181.96 84.46) (width 0.2) (layer "F.Cu") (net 14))
 (segment (start 181.805 102.5) (end 181.805 97.615) (width 0.2) (layer "F.Cu") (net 14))
 (segment (start 181.61 97.42) (end 184.5 94.53) (width 0.2) (layer "F.Cu") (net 14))
 (segment (start 184.5 87) (end 189.425 87) (width 0.2) (layer "F.Cu") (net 14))
 (segment (start 184.5 94.53) (end 184.5 87) (width 0.2) (layer "F.Cu") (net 14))
 (segment (start 181.96 84.46) (end 184.5 87) (width 0.2) (layer "F.Cu") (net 14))
 (segment (start 249.54 85.7575) (end 242.5325 78.75) (width 0.2) (layer "F.Cu") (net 6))
 (segment (start 242.5325 78.75) (end 233.62 78.75) (width 0.2) (layer "F.Cu") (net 6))
 (segment (start 249.5225 83.2) (end 252.08 85.7575) (width 0.2) (layer "B.Cu") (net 32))
 (segment (start 249.5225 83.2) (end 236 83.2) (width 0.2) (layer "B.Cu") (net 32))
 (segment (start 236 87.25) (end 249.54 100.79) (width 0.2) (layer "F.Cu") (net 27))
 (segment (start 249.54 100.79) (end 249.54 100.9975) (width 0.2) (layer "F.Cu") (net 27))
 (segment (start 236 92.5375) (end 244.46 100.9975) (width 0.2) (layer "F.Cu") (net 36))
 (segment (start 236 91.3) (end 236 92.5375) (width 0.2) (layer "F.Cu") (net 36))
 (segment (start 236.2725 95.35) (end 241.92 100.9975) (width 0.2) (layer "F.Cu") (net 34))
 (segment (start 244.46 90.94) (end 244.46 85.7575) (width 0.2) (layer "B.Cu") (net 29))
 (segment (start 236 99.4) (end 244.46 90.94) (width 0.2) (layer "B.Cu") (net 29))
 (segment (start 233.5 101) (end 233.5 99.40705) (width 0.2) (layer "B.Cu") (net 25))
 (segment (start 233.5 99.40705) (end 241.92 90.98705) (width 0.2) (layer "B.Cu") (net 25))
 (segment (start 235.95 103.45) (end 233.5 101) (width 0.2) (layer "B.Cu") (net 25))
 (segment (start 241.92 90.98705) (end 241.92 85.7575) (width 0.2) (layer "B.Cu") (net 25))
 (segment (start 236 103.45) (end 235.95 103.45) (width 0.2) (layer "B.Cu") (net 25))
 (segment (start 236 107.5) (end 245.5775 107.5) (width 0.2) (layer "F.Cu") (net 37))
 (segment (start 245.5775 107.5) (end 252.08 100.9975) (width 0.2) (layer "F.Cu") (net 37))
 (segment (start 170 100.96) (end 173 97.96) (width 0.2) (layer "F.Cu") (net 7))
 (segment (start 173 91) (end 170 88) (width 0.2) (layer "F.Cu") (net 7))
 (segment (start 173 97.96) (end 173 91) (width 0.2) (layer "F.Cu") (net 7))
 (segment (start 205.63137 89.5) (end 204.5 89.5) (width 0.2) (layer "F.Cu") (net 10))
 (segment (start 213 96) (end 213 97.2) (width 0.2) (layer "F.Cu") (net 10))
 (segment (start 196.88 84.42) (end 199.42 84.42) (width 0.2) (layer "F.Cu") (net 10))
 (segment (start 213 96) (end 212.059 95.059) (width 0.2) (layer "F.Cu") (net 10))
 (segment (start 211.19037 95.059) (end 205.63137 89.5) (width 0.2) (layer "F.Cu") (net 10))
 (segment (start 213 97.2) (end 211.5 98.7) (width 0.2) (layer "F.Cu") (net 10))
 (segment (start 212.059 95.059) (end 211.19037 95.059) (width 0.2) (layer "F.Cu") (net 10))
 (segment (start 199.42 84.42) (end 204.5 89.5) (width 0.2) (layer "F.Cu") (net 10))
 (segment (start 204.5 92.04) (end 207.38 92.04) (width 0.2) (layer "F.Cu") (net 13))
 (segment (start 207.38 92.04) (end 211.5 96.16) (width 0.2) (layer "F.Cu") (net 13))
 (segment (start 207.5 87) (end 211.04 83.46) (width 0.2) (layer "B.Cu") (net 12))
 (segment (start 211.04 83.46) (end 211.5 83.46) (width 0.2) (layer "B.Cu") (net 12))
 (segment (start 207.5 94.12) (end 207.5 87) (width 0.2) (layer "B.Cu") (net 12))
 (segment (start 204.5 97.12) (end 207.5 94.12) (width 0.2) (layer "B.Cu") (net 12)))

